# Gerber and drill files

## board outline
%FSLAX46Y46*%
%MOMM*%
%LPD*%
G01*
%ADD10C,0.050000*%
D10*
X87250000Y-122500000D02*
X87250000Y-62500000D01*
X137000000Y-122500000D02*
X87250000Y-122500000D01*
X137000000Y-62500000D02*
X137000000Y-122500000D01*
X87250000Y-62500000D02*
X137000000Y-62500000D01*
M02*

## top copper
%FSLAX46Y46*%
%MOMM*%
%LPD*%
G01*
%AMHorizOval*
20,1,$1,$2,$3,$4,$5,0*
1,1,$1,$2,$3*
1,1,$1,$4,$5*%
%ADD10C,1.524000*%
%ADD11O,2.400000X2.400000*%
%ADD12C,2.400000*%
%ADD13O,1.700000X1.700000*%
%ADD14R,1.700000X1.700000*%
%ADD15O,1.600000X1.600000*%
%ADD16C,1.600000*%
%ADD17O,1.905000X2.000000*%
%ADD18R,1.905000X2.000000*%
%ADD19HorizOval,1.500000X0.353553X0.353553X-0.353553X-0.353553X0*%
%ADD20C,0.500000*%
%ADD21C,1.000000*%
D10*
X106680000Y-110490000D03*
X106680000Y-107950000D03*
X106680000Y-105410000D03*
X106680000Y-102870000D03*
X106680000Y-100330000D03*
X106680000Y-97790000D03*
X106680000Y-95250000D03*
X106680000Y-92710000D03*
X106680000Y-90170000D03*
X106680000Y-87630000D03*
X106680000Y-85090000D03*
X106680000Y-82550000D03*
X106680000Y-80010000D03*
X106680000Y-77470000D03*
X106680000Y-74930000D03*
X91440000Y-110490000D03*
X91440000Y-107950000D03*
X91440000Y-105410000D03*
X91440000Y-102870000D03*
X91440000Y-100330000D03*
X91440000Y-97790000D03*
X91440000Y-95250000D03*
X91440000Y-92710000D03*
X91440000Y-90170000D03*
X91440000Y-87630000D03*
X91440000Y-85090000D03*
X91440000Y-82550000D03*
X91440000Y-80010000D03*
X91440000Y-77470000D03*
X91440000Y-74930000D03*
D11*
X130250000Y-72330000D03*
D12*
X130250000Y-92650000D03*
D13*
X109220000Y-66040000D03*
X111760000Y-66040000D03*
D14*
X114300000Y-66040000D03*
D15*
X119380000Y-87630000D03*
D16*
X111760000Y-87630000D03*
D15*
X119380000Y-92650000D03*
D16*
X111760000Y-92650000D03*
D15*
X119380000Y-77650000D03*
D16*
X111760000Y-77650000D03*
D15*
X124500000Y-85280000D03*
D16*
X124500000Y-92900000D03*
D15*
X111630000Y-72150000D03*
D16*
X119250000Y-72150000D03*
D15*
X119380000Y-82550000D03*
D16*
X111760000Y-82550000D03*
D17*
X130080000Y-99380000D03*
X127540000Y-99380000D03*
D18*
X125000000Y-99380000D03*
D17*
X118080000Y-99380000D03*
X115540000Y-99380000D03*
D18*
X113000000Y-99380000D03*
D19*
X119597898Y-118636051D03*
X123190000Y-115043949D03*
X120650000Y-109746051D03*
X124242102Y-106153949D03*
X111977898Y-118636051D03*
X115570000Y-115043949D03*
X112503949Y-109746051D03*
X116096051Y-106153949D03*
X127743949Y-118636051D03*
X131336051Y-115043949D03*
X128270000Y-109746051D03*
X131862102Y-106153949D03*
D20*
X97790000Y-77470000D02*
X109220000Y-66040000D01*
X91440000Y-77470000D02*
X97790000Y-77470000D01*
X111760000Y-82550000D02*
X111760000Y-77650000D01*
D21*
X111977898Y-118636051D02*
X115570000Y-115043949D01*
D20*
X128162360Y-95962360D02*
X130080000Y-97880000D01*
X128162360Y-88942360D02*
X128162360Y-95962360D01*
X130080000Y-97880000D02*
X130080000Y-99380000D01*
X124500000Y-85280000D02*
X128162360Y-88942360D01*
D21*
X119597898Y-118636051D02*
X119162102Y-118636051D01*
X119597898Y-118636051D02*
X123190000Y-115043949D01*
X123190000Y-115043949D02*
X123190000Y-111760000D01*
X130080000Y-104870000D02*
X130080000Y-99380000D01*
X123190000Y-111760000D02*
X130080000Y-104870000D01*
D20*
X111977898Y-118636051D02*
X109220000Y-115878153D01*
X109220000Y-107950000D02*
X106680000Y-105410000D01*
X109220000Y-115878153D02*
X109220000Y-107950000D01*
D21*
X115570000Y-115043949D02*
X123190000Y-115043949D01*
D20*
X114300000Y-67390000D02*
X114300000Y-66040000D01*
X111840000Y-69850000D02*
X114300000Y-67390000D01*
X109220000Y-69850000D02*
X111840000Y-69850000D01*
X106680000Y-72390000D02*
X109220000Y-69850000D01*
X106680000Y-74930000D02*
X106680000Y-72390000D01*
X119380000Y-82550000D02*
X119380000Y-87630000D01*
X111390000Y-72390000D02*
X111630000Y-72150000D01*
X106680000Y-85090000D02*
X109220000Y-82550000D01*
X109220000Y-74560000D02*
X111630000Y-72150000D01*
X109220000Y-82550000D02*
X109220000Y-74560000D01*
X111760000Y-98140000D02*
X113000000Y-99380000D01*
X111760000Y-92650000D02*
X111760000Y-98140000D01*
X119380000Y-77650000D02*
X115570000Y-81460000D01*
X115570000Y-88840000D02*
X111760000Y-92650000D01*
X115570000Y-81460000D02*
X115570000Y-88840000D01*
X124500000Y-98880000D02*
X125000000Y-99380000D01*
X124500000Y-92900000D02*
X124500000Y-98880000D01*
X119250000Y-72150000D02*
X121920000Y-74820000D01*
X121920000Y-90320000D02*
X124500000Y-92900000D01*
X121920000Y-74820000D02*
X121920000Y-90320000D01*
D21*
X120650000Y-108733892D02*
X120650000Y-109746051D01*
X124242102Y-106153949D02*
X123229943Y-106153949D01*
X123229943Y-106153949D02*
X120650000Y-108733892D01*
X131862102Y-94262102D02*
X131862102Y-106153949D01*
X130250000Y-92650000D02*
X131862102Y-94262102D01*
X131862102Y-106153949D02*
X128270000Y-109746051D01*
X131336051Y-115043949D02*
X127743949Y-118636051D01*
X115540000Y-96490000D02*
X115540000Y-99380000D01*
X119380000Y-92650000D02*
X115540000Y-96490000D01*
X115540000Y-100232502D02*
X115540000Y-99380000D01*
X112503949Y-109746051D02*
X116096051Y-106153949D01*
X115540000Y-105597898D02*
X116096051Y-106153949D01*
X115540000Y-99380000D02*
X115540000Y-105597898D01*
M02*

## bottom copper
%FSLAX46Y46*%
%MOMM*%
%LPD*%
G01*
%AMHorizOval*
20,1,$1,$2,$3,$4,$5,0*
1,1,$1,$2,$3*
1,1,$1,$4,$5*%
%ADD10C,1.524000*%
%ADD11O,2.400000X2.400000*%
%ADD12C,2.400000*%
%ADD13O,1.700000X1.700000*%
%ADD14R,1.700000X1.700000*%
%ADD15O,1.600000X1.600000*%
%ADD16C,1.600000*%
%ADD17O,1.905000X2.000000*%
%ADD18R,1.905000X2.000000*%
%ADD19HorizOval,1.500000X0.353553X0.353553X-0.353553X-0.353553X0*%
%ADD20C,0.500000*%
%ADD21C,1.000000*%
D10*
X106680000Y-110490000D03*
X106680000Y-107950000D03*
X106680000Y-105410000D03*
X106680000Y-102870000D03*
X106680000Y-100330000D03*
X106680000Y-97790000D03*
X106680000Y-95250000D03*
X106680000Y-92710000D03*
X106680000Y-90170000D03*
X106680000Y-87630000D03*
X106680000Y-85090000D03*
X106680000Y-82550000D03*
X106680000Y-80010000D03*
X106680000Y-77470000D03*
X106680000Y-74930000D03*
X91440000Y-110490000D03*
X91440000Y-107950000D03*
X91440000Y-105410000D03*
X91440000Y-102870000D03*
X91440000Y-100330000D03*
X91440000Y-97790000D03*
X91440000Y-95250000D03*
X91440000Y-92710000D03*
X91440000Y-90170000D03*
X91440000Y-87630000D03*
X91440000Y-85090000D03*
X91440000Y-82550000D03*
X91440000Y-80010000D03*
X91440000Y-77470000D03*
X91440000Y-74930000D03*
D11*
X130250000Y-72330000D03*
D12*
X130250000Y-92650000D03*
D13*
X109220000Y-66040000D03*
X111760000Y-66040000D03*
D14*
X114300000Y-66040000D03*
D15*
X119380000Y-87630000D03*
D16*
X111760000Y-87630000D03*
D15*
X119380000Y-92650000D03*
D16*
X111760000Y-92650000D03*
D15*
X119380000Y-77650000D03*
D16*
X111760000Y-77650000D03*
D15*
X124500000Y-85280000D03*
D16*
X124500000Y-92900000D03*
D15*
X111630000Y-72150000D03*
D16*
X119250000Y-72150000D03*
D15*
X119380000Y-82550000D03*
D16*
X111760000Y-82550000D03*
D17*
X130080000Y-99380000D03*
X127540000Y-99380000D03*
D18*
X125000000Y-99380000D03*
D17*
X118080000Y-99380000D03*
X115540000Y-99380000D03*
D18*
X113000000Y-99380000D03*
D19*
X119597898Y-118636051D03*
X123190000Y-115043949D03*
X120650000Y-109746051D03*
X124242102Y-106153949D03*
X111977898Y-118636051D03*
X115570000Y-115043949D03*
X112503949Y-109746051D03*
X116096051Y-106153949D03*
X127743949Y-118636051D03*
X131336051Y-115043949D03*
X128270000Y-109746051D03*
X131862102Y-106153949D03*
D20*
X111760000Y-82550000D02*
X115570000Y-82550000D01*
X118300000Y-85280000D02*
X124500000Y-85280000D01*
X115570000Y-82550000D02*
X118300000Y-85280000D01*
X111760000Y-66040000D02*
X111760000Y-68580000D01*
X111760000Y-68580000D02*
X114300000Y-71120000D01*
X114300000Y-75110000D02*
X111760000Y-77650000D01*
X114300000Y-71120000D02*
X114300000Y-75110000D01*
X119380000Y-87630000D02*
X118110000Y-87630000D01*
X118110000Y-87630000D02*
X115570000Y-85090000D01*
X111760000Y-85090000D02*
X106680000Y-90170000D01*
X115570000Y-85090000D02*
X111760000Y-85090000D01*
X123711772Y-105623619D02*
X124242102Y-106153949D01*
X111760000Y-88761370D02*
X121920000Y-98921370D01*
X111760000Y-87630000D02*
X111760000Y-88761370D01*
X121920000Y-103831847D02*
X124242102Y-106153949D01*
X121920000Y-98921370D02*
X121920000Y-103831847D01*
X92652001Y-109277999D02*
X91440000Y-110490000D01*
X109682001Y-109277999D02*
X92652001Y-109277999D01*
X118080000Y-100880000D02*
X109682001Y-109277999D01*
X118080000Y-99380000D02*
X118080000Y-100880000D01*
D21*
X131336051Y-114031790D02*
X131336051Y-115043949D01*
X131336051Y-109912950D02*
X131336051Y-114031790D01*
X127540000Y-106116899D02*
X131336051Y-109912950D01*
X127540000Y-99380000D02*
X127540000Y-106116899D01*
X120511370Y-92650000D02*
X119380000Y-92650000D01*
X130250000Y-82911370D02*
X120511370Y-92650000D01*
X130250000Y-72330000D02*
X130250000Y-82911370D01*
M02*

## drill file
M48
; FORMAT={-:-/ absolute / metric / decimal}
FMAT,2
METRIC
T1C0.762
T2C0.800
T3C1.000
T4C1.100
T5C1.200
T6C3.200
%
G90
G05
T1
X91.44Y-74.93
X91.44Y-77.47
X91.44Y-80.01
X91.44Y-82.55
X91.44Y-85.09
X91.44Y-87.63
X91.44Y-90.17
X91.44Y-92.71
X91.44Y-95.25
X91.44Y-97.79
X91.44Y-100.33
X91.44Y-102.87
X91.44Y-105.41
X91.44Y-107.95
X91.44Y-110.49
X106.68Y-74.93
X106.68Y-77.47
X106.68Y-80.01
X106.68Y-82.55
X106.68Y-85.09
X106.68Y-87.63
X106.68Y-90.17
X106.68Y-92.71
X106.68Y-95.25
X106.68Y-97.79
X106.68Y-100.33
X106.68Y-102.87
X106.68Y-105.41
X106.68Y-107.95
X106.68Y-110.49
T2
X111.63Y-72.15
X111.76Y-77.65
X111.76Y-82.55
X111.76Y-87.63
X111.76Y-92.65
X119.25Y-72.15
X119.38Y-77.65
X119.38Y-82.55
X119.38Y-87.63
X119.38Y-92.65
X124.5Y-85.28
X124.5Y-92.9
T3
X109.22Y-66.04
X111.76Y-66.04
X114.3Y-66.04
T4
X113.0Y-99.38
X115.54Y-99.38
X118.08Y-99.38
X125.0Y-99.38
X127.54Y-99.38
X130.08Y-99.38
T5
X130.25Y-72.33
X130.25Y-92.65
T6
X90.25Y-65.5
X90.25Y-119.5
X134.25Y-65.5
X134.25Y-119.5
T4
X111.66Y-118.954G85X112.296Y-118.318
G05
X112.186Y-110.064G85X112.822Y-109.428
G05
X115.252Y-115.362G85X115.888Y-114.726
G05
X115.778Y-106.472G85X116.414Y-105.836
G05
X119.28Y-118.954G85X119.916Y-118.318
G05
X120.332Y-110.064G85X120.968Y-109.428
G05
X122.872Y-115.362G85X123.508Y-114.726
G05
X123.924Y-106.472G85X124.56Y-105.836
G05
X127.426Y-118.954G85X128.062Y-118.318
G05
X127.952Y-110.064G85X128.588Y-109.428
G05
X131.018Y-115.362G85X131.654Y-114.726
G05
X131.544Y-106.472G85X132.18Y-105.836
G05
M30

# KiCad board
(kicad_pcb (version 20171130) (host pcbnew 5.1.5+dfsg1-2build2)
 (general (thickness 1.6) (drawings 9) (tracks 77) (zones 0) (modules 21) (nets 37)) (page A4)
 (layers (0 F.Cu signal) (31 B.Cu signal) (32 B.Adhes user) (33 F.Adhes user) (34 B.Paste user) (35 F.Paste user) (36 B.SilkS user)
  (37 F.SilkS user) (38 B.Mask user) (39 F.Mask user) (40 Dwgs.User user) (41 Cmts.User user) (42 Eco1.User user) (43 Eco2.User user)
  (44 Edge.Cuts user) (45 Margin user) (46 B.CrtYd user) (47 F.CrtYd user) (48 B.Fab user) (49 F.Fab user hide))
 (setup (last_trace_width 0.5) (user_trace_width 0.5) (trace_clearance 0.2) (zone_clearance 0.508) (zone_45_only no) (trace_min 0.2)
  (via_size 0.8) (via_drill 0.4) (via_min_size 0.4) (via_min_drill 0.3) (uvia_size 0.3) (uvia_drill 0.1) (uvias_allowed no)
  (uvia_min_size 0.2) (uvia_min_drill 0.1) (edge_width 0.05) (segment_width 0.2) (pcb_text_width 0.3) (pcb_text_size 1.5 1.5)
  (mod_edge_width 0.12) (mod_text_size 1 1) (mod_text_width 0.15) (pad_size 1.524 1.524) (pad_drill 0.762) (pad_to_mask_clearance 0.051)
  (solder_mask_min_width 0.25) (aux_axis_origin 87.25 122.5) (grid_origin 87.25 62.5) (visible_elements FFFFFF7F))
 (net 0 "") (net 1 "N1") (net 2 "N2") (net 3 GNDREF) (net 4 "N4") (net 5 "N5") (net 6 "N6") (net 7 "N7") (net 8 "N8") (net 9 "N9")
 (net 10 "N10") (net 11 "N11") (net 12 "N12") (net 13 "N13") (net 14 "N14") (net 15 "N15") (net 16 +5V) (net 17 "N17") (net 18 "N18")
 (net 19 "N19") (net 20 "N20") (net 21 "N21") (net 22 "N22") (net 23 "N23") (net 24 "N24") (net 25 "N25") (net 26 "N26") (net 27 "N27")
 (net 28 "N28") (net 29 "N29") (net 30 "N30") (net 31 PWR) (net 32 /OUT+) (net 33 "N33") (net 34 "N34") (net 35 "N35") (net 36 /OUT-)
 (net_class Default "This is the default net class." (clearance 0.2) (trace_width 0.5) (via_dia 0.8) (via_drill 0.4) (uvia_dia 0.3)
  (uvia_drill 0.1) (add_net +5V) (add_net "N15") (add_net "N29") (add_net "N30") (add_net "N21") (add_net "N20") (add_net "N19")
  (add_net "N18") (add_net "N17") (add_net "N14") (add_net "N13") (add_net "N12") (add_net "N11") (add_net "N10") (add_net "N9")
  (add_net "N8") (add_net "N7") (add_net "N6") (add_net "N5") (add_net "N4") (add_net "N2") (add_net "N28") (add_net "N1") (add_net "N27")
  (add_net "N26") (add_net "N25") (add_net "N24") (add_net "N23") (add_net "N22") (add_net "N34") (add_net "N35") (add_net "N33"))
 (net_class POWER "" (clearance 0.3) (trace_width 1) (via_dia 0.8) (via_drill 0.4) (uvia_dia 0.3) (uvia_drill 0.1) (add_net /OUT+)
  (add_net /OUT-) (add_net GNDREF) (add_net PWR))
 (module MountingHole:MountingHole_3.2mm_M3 (layer F.Cu) (at 90.25 119.5)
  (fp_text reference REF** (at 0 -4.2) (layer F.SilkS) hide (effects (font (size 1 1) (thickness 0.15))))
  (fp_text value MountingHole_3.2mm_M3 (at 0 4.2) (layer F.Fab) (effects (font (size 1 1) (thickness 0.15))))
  (pad 1 np_thru_hole circle (at 0 0) (size 3.2 3.2) (drill 3.2) (layers *.Cu *.Mask)))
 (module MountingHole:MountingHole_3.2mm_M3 (layer F.Cu) (at 134.25 119.5)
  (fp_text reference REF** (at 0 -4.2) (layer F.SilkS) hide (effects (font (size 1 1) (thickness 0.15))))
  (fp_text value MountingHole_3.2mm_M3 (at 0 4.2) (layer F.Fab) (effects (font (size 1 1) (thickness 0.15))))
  (pad 1 np_thru_hole circle (at 0 0) (size 3.2 3.2) (drill 3.2) (layers *.Cu *.Mask)))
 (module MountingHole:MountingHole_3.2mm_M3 (layer F.Cu) (at 134.25 65.5)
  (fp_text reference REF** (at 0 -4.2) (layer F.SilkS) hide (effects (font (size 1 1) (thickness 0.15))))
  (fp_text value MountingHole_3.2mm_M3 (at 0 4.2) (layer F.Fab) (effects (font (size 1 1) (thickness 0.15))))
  (pad 1 np_thru_hole circle (at 0 0) (size 3.2 3.2) (drill 3.2) (layers *.Cu *.Mask)))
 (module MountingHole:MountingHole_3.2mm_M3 (layer F.Cu) (at 90.25 65.5)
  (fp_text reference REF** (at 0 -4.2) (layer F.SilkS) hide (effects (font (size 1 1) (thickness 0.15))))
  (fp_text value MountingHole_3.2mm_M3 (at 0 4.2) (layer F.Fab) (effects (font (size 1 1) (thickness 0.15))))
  (pad 1 np_thru_hole circle (at 0 0) (size 3.2 3.2) (drill 3.2) (layers *.Cu *.Mask)))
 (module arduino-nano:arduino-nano (layer F.Cu) (at 99.06 92.71)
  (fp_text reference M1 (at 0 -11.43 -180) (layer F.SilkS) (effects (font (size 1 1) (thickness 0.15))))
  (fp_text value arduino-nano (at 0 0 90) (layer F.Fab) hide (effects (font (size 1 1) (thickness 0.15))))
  (pad 30 thru_hole circle (at 7.62 17.78) (size 1.524 1.524) (drill 0.762) (layers *.Cu *.Mask) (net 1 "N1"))
  (pad 29 thru_hole circle (at 7.62 15.24) (size 1.524 1.524) (drill 0.762) (layers *.Cu *.Mask) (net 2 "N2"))
  (pad 28 thru_hole circle (at 7.62 12.7) (size 1.524 1.524) (drill 0.762) (layers *.Cu *.Mask) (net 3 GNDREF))
  (pad 27 thru_hole circle (at 7.62 10.16) (size 1.524 1.524) (drill 0.762) (layers *.Cu *.Mask) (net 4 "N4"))
  (pad 26 thru_hole circle (at 7.62 7.62) (size 1.524 1.524) (drill 0.762) (layers *.Cu *.Mask) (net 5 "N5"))
  (pad 25 thru_hole circle (at 7.62 5.08) (size 1.524 1.524) (drill 0.762) (layers *.Cu *.Mask) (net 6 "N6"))
  (pad 24 thru_hole circle (at 7.62 2.54) (size 1.524 1.524) (drill 0.762) (layers *.Cu *.Mask) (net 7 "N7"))
  (pad 23 thru_hole circle (at 7.62 0) (size 1.524 1.524) (drill 0.762) (layers *.Cu *.Mask) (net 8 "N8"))
  (pad 22 thru_hole circle (at 7.62 -2.54) (size 1.524 1.524) (drill 0.762) (layers *.Cu *.Mask) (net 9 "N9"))
  (pad 21 thru_hole circle (at 7.62 -5.08) (size 1.524 1.524) (drill 0.762) (layers *.Cu *.Mask) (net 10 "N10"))
  (pad 20 thru_hole circle (at 7.62 -7.62) (size 1.524 1.524) (drill 0.762) (layers *.Cu *.Mask) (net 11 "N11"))
  (pad 19 thru_hole circle (at 7.62 -10.16) (size 1.524 1.524) (drill 0.762) (layers *.Cu *.Mask) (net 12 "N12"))
  (pad 18 thru_hole circle (at 7.62 -12.7) (size 1.524 1.524) (drill 0.762) (layers *.Cu *.Mask) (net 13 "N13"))
  (pad 17 thru_hole circle (at 7.62 -15.24) (size 1.524 1.524) (drill 0.762) (layers *.Cu *.Mask) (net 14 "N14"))
  (pad 16 thru_hole circle (at 7.62 -17.78) (size 1.524 1.524) (drill 0.762) (layers *.Cu *.Mask) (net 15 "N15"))
  (pad 15 thru_hole circle (at -7.62 17.78) (size 1.524 1.524) (drill 0.762) (layers *.Cu *.Mask) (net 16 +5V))
  (pad 14 thru_hole circle (at -7.62 15.24) (size 1.524 1.524) (drill 0.762) (layers *.Cu *.Mask) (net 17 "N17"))
  (pad 13 thru_hole circle (at -7.62 12.7) (size 1.524 1.524) (drill 0.762) (layers *.Cu *.Mask) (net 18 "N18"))
  (pad 12 thru_hole circle (at -7.62 10.16) (size 1.524 1.524) (drill 0.762) (layers *.Cu *.Mask) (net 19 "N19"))
  (pad 11 thru_hole circle (at -7.62 7.62) (size 1.524 1.524) (drill 0.762) (layers *.Cu *.Mask) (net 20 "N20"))
  (pad 10 thru_hole circle (at -7.62 5.08) (size 1.524 1.524) (drill 0.762) (layers *.Cu *.Mask) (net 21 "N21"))
  (pad 9 thru_hole circle (at -7.62 2.54) (size 1.524 1.524) (drill 0.762) (layers *.Cu *.Mask) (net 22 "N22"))
  (pad 8 thru_hole circle (at -7.62 0) (size 1.524 1.524) (drill 0.762) (layers *.Cu *.Mask) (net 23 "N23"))
  (pad 7 thru_hole circle (at -7.62 -2.54) (size 1.524 1.524) (drill 0.762) (layers *.Cu *.Mask) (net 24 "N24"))
  (pad 6 thru_hole circle (at -7.62 -5.08) (size 1.524 1.524) (drill 0.762) (layers *.Cu *.Mask) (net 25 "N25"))
  (pad 5 thru_hole circle (at -7.62 -7.62) (size 1.524 1.524) (drill 0.762) (layers *.Cu *.Mask) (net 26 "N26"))
  (pad 4 thru_hole circle (at -7.62 -10.16) (size 1.524 1.524) (drill 0.762) (layers *.Cu *.Mask) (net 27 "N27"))
  (pad 3 thru_hole circle (at -7.62 -12.7) (size 1.524 1.524) (drill 0.762) (layers *.Cu *.Mask) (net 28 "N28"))
  (pad 2 thru_hole circle (at -7.62 -15.24) (size 1.524 1.524) (drill 0.762) (layers *.Cu *.Mask) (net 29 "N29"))
  (pad 1 thru_hole circle (at -7.62 -17.78) (size 1.524 1.524) (drill 0.762) (layers *.Cu *.Mask) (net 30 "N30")))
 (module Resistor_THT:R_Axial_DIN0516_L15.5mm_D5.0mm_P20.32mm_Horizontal (layer F.Cu) (at 130.25 92.65 90)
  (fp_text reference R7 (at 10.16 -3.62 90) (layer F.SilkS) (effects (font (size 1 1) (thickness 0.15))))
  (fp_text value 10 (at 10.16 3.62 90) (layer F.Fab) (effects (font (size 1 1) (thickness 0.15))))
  (pad 2 thru_hole oval (at 20.32 0 90) (size 2.4 2.4) (drill 1.2) (layers *.Cu *.Mask) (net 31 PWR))
  (pad 1 thru_hole circle (at 0 0 90) (size 2.4 2.4) (drill 1.2) (layers *.Cu *.Mask) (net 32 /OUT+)))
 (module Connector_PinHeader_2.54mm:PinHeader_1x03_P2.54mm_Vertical (layer F.Cu) (at 114.3 66.04 270)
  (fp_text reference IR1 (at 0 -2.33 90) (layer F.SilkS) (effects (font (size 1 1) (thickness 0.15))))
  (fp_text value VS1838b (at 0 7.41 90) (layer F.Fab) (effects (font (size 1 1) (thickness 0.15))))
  (pad 3 thru_hole oval (at 0 5.08 270) (size 1.7 1.7) (drill 1) (layers *.Cu *.Mask) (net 29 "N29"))
  (pad 2 thru_hole oval (at 0 2.54 270) (size 1.7 1.7) (drill 1) (layers *.Cu *.Mask) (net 3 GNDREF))
  (pad 1 thru_hole rect (at 0 0 270) (size 1.7 1.7) (drill 1) (layers *.Cu *.Mask) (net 15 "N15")))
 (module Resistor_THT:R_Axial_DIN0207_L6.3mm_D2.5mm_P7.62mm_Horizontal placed (layer F.Cu) (at 111.76 87.63)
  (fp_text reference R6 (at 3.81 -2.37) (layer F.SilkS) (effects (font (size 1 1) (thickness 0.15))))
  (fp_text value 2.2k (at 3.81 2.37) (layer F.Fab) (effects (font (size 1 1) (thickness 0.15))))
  (pad 2 thru_hole oval (at 7.62 0) (size 1.6 1.6) (drill 0.8) (layers *.Cu *.Mask) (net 9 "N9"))
  (pad 1 thru_hole circle (at 0 0) (size 1.6 1.6) (drill 0.8) (layers *.Cu *.Mask) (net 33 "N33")))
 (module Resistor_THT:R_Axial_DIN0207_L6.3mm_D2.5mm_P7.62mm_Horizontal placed (layer F.Cu) (at 111.76 92.65)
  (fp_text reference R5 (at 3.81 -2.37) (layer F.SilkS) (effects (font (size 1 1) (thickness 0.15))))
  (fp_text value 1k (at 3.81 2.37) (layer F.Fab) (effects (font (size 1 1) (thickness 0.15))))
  (pad 2 thru_hole oval (at 7.62 0) (size 1.6 1.6) (drill 0.8) (layers *.Cu *.Mask) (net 31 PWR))
  (pad 1 thru_hole circle (at 0 0) (size 1.6 1.6) (drill 0.8) (layers *.Cu *.Mask) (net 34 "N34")))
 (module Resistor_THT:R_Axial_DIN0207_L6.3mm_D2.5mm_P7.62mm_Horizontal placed (layer F.Cu) (at 111.76 77.65)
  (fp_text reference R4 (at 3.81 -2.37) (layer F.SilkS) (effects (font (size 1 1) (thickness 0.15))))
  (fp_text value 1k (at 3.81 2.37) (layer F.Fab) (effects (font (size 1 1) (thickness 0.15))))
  (pad 2 thru_hole oval (at 7.62 0) (size 1.6 1.6) (drill 0.8) (layers *.Cu *.Mask) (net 34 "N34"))
  (pad 1 thru_hole circle (at 0 0) (size 1.6 1.6) (drill 0.8) (layers *.Cu *.Mask) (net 3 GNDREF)))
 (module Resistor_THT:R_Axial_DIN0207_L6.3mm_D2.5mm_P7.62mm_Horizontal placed (layer F.Cu) (at 124.5 92.9 90)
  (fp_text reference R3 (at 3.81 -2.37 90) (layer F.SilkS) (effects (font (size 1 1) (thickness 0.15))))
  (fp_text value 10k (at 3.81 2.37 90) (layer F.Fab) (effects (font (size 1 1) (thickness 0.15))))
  (pad 2 thru_hole oval (at 7.62 0 90) (size 1.6 1.6) (drill 0.8) (layers *.Cu *.Mask) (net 3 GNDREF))
  (pad 1 thru_hole circle (at 0 0 90) (size 1.6 1.6) (drill 0.8) (layers *.Cu *.Mask) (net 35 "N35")))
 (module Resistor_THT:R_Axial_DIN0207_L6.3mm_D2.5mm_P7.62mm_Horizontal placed (layer F.Cu) (at 119.25 72.15 180)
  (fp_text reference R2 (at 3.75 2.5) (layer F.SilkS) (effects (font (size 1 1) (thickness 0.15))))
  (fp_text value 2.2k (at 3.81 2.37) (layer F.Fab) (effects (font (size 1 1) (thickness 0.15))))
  (pad 2 thru_hole oval (at 7.62 0 180) (size 1.6 1.6) (drill 0.8) (layers *.Cu *.Mask) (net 11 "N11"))
  (pad 1 thru_hole circle (at 0 0 180) (size 1.6 1.6) (drill 0.8) (layers *.Cu *.Mask) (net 35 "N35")))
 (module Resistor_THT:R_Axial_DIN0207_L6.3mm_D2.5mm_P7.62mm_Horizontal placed (layer F.Cu) (at 111.76 82.55)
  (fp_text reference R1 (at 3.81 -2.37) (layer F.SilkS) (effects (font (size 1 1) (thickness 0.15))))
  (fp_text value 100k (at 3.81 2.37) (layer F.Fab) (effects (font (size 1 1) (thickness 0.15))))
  (pad 2 thru_hole oval (at 7.62 0) (size 1.6 1.6) (drill 0.8) (layers *.Cu *.Mask) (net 9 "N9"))
  (pad 1 thru_hole circle (at 0 0) (size 1.6 1.6) (drill 0.8) (layers *.Cu *.Mask) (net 3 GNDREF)))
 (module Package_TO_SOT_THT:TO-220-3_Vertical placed (layer F.Cu) (at 125 99.38)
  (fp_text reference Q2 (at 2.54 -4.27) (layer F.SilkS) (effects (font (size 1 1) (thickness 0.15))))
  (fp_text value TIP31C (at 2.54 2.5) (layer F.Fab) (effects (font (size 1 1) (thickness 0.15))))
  (pad 3 thru_hole oval (at 5.08 0) (size 1.905 2) (drill 1.1) (layers *.Cu *.Mask) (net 3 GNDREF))
  (pad 2 thru_hole oval (at 2.54 0) (size 1.905 2) (drill 1.1) (layers *.Cu *.Mask) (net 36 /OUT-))
  (pad 1 thru_hole rect (at 0 0) (size 1.905 2) (drill 1.1) (layers *.Cu *.Mask) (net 35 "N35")))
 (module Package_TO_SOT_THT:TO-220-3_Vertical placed (layer F.Cu) (at 113 99.38)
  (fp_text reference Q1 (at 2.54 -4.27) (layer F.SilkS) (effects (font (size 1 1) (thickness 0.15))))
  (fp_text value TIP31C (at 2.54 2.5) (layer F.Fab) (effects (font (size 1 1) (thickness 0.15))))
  (pad 3 thru_hole oval (at 5.08 0) (size 1.905 2) (drill 1.1) (layers *.Cu *.Mask) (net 16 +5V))
  (pad 2 thru_hole oval (at 2.54 0) (size 1.905 2) (drill 1.1) (layers *.Cu *.Mask) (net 31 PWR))
  (pad 1 thru_hole rect (at 0 0) (size 1.905 2) (drill 1.1) (layers *.Cu *.Mask) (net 34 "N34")))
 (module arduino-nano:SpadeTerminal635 (layer F.Cu) (at 121.393949 116.84 45)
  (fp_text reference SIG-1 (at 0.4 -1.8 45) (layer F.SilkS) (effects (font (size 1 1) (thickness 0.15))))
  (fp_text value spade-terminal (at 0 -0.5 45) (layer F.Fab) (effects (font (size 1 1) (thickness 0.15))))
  (pad 1 thru_hole oval (at -2.54 0 45) (size 2.5 1.5) (drill oval 2 1.1) (layers *.Cu *.Mask) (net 3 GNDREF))
  (pad 1 thru_hole oval (at 2.54 0 45) (size 2.5 1.5) (drill oval 2 1.1) (layers *.Cu *.Mask) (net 3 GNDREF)))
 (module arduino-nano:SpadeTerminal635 (layer F.Cu) (at 122.446051 107.95 45)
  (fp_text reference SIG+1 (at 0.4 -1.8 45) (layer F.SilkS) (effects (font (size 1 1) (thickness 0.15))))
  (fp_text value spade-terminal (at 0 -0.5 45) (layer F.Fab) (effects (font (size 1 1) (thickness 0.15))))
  (pad 1 thru_hole oval (at -2.54 0 45) (size 2.5 1.5) (drill oval 2 1.1) (layers *.Cu *.Mask) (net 33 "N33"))
  (pad 1 thru_hole oval (at 2.54 0 45) (size 2.5 1.5) (drill oval 2 1.1) (layers *.Cu *.Mask) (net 33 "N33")))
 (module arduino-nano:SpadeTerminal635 (layer F.Cu) (at 113.773949 116.84 45)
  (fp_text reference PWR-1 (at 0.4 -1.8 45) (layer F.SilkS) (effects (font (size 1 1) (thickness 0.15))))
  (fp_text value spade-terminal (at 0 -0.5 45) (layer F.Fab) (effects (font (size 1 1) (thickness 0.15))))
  (pad 1 thru_hole oval (at -2.54 0 45) (size 2.5 1.5) (drill oval 2 1.1) (layers *.Cu *.Mask) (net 3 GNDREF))
  (pad 1 thru_hole oval (at 2.54 0 45) (size 2.5 1.5) (drill oval 2 1.1) (layers *.Cu *.Mask) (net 3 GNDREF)))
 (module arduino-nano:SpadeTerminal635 (layer F.Cu) (at 114.3 107.95 45)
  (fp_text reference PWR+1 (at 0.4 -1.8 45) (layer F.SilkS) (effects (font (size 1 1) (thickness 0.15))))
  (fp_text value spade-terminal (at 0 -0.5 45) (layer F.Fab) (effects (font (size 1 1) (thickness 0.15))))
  (pad 1 thru_hole oval (at -2.54 0 45) (size 2.5 1.5) (drill oval 2 1.1) (layers *.Cu *.Mask) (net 31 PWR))
  (pad 1 thru_hole oval (at 2.54 0 45) (size 2.5 1.5) (drill oval 2 1.1) (layers *.Cu *.Mask) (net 31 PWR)))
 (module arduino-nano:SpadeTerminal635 (layer F.Cu) (at 129.54 116.84 45)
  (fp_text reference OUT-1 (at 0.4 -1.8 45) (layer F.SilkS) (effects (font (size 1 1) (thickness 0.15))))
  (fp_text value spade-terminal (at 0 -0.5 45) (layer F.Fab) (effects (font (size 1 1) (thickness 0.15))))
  (pad 1 thru_hole oval (at -2.54 0 45) (size 2.5 1.5) (drill oval 2 1.1) (layers *.Cu *.Mask) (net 36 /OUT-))
  (pad 1 thru_hole oval (at 2.54 0 45) (size 2.5 1.5) (drill oval 2 1.1) (layers *.Cu *.Mask) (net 36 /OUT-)))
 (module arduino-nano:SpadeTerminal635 (layer F.Cu) (at 130.066051 107.95 45)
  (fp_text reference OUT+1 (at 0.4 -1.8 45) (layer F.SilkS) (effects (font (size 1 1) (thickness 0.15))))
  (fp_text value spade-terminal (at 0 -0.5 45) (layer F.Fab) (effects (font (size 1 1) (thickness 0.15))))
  (pad 1 thru_hole oval (at -2.54 0 45) (size 2.5 1.5) (drill oval 2 1.1) (layers *.Cu *.Mask) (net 32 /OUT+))
  (pad 1 thru_hole oval (at 2.54 0 45) (size 2.5 1.5) (drill oval 2 1.1) (layers *.Cu *.Mask) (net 32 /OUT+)))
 (gr_line (start 87.25 122.5) (end 87.25 62.5) (layer Edge.Cuts) (width 0.05))
 (gr_line (start 137 122.5) (end 87.25 122.5) (layer Edge.Cuts) (width 0.05))
 (gr_line (start 137 62.5) (end 137 122.5) (layer Edge.Cuts) (width 0.05))
 (gr_line (start 87.25 62.5) (end 137 62.5) (layer Edge.Cuts) (width 0.05))
 (segment (start 97.79 77.47) (end 109.22 66.04) (width 0.5) (layer F.Cu) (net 29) (status 20))
 (segment (start 91.44 77.47) (end 97.79 77.47) (width 0.5) (layer F.Cu) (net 29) (status 10))
 (segment (start 111.76 82.55) (end 111.76 77.65) (width 0.5) (layer F.Cu) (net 3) (status 30))
 (segment (start 111.977898 118.636051) (end 115.57 115.043949) (width 1) (layer F.Cu) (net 3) (status 30))
 (segment (start 128.16236 95.96236) (end 130.08 97.88) (width 0.5) (layer F.Cu) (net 3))
 (segment (start 128.16236 88.94236) (end 128.16236 95.96236) (width 0.5) (layer F.Cu) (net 3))
 (segment (start 130.08 97.88) (end 130.08 99.38) (width 0.5) (layer F.Cu) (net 3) (status 20))
 (segment (start 124.5 85.28) (end 128.16236 88.94236) (width 0.5) (layer F.Cu) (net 3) (status 10))
 (segment (start 119.597898 118.636051) (end 119.162102 118.636051) (width 1) (layer F.Cu) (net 3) (status 30))
 (segment (start 119.597898 118.636051) (end 123.19 115.043949) (width 1) (layer F.Cu) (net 3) (status 30))
 (segment (start 123.19 115.043949) (end 123.19 111.76) (width 1) (layer F.Cu) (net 3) (status 10))
 (segment (start 130.08 104.87) (end 130.08 99.38) (width 1) (layer F.Cu) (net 3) (status 20))
 (segment (start 123.19 111.76) (end 130.08 104.87) (width 1) (layer F.Cu) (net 3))
 (segment (start 111.76 82.55) (end 115.57 82.55) (width 0.5) (layer B.Cu) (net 3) (status 10))
 (segment (start 118.3 85.28) (end 124.5 85.28) (width 0.5) (layer B.Cu) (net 3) (status 20))
 (segment (start 115.57 82.55) (end 118.3 85.28) (width 0.5) (layer B.Cu) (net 3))
 (segment (start 111.76 66.04) (end 111.76 68.58) (width 0.5) (layer B.Cu) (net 3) (status 10))
 (segment (start 111.76 68.58) (end 114.3 71.12) (width 0.5) (layer B.Cu) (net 3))
 (segment (start 114.3 75.11) (end 111.76 77.65) (width 0.5) (layer B.Cu) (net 3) (status 20))
 (segment (start 114.3 71.12) (end 114.3 75.11) (width 0.5) (layer B.Cu) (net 3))
 (segment (start 111.977898 118.636051) (end 109.22 115.878153) (width 0.5) (layer F.Cu) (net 3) (status 10))
 (segment (start 109.22 107.95) (end 106.68 105.41) (width 0.5) (layer F.Cu) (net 3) (status 20))
 (segment (start 109.22 115.878153) (end 109.22 107.95) (width 0.5) (layer F.Cu) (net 3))
 (segment (start 115.57 115.043949) (end 123.19 115.043949) (width 1) (layer F.Cu) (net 3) (status 30))
 (segment (start 114.3 67.39) (end 114.3 66.04) (width 0.5) (layer F.Cu) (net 15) (status 20))
 (segment (start 111.84 69.85) (end 114.3 67.39) (width 0.5) (layer F.Cu) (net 15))
 (segment (start 109.22 69.85) (end 111.84 69.85) (width 0.5) (layer F.Cu) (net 15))
 (segment (start 106.68 72.39) (end 109.22 69.85) (width 0.5) (layer F.Cu) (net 15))
 (segment (start 106.68 74.93) (end 106.68 72.39) (width 0.5) (layer F.Cu) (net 15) (status 10))
 (segment (start 119.38 82.55) (end 119.38 87.63) (width 0.5) (layer F.Cu) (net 9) (status 30))
 (segment (start 119.38 87.63) (end 118.11 87.63) (width 0.5) (layer B.Cu) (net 9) (status 10))
 (segment (start 118.11 87.63) (end 115.57 85.09) (width 0.5) (layer B.Cu) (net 9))
 (segment (start 111.76 85.09) (end 106.68 90.17) (width 0.5) (layer B.Cu) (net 9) (status 20))
 (segment (start 115.57 85.09) (end 111.76 85.09) (width 0.5) (layer B.Cu) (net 9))
 (segment (start 111.39 72.39) (end 111.63 72.15) (width 0.5) (layer F.Cu) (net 11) (status 30))
 (segment (start 106.68 85.09) (end 109.22 82.55) (width 0.5) (layer F.Cu) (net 11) (status 10))
 (segment (start 109.22 74.56) (end 111.63 72.15) (width 0.5) (layer F.Cu) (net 11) (status 20))
 (segment (start 109.22 82.55) (end 109.22 74.56) (width 0.5) (layer F.Cu) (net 11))
 (segment (start 111.76 98.14) (end 113 99.38) (width 0.5) (layer F.Cu) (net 34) (status 20))
 (segment (start 111.76 92.65) (end 111.76 98.14) (width 0.5) (layer F.Cu) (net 34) (status 10))
 (segment (start 119.38 77.65) (end 115.57 81.46) (width 0.5) (layer F.Cu) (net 34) (status 10))
 (segment (start 115.57 88.84) (end 111.76 92.65) (width 0.5) (layer F.Cu) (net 34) (status 20))
 (segment (start 115.57 81.46) (end 115.57 88.84) (width 0.5) (layer F.Cu) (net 34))
 (segment (start 124.5 98.88) (end 125 99.38) (width 0.5) (layer F.Cu) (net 35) (status 30))
 (segment (start 124.5 92.9) (end 124.5 98.88) (width 0.5) (layer F.Cu) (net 35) (status 30))
 (segment (start 119.25 72.15) (end 121.92 74.82) (width 0.5) (layer F.Cu) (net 35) (status 10))
 (segment (start 121.92 90.32) (end 124.5 92.9) (width 0.5) (layer F.Cu) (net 35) (status 20))
 (segment (start 121.92 74.82) (end 121.92 90.32) (width 0.5) (layer F.Cu) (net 35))
 (segment (start 123.711772 105.623619) (end 124.242102 106.153949) (width 0.5) (layer B.Cu) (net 33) (status 30))
 (segment (start 111.76 88.76137) (end 121.92 98.92137) (width 0.5) (layer B.Cu) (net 33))
 (segment (start 111.76 87.63) (end 111.76 88.76137) (width 0.5) (layer B.Cu) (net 33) (status 10))
 (segment (start 121.92 103.831847) (end 124.242102 106.153949) (width 0.5) (layer B.Cu) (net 33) (status 20))
 (segment (start 121.92 98.92137) (end 121.92 103.831847) (width 0.5) (layer B.Cu) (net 33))
 (segment (start 120.65 108.733892) (end 120.65 109.746051) (width 1) (layer F.Cu) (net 33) (status 30))
 (segment (start 124.242102 106.153949) (end 123.229943 106.153949) (width 1) (layer F.Cu) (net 33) (status 30))
 (segment (start 123.229943 106.153949) (end 120.65 108.733892) (width 1) (layer F.Cu) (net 33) (status 30))
 (segment (start 92.652001 109.277999) (end 91.44 110.49) (width 0.5) (layer B.Cu) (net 16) (status 20))
 (segment (start 109.682001 109.277999) (end 92.652001 109.277999) (width 0.5) (layer B.Cu) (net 16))
 (segment (start 118.08 100.88) (end 109.682001 109.277999) (width 0.5) (layer B.Cu) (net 16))
 (segment (start 118.08 99.38) (end 118.08 100.88) (width 0.5) (layer B.Cu) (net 16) (status 10))
 (segment (start 131.862102 94.262102) (end 131.862102 106.153949) (width 1) (layer F.Cu) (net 32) (status 20))
 (segment (start 130.25 92.65) (end 131.862102 94.262102) (width 1) (layer F.Cu) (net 32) (status 10))
 (segment (start 131.862102 106.153949) (end 128.27 109.746051) (width 1) (layer F.Cu) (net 32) (status 30))
 (segment (start 131.336051 115.043949) (end 127.743949 118.636051) (width 1) (layer F.Cu) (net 36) (status 30))
 (segment (start 131.336051 114.03179) (end 131.336051 115.043949) (width 1) (layer B.Cu) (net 36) (status 30))
 (segment (start 131.336051 109.91295) (end 131.336051 114.03179) (width 1) (layer B.Cu) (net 36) (status 20))
 (segment (start 127.54 106.116899) (end 131.336051 109.91295) (width 1) (layer B.Cu) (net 36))
 (segment (start 127.54 99.38) (end 127.54 106.116899) (width 1) (layer B.Cu) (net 36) (status 10))
 (segment (start 115.54 96.49) (end 115.54 99.38) (width 1) (layer F.Cu) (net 31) (status 20))
 (segment (start 119.38 92.65) (end 115.54 96.49) (width 1) (layer F.Cu) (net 31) (status 10))
 (segment (start 115.54 100.232502) (end 115.54 99.38) (width 1) (layer F.Cu) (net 31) (status 30))
 (segment (start 120.51137 92.65) (end 119.38 92.65) (width 1) (layer B.Cu) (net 31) (status 20))
 (segment (start 130.25 82.91137) (end 120.51137 92.65) (width 1) (layer B.Cu) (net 31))
 (segment (start 130.25 72.33) (end 130.25 82.91137) (width 1) (layer B.Cu) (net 31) (status 10))
 (segment (start 112.503949 109.746051) (end 116.096051 106.153949) (width 1) (layer F.Cu) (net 31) (status 30))
 (segment (start 115.54 105.597898) (end 116.096051 106.153949) (width 1) (layer F.Cu) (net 31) (status 20))
 (segment (start 115.54 99.38) (end 115.54 105.597898) (width 1) (layer F.Cu) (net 31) (status 10)))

